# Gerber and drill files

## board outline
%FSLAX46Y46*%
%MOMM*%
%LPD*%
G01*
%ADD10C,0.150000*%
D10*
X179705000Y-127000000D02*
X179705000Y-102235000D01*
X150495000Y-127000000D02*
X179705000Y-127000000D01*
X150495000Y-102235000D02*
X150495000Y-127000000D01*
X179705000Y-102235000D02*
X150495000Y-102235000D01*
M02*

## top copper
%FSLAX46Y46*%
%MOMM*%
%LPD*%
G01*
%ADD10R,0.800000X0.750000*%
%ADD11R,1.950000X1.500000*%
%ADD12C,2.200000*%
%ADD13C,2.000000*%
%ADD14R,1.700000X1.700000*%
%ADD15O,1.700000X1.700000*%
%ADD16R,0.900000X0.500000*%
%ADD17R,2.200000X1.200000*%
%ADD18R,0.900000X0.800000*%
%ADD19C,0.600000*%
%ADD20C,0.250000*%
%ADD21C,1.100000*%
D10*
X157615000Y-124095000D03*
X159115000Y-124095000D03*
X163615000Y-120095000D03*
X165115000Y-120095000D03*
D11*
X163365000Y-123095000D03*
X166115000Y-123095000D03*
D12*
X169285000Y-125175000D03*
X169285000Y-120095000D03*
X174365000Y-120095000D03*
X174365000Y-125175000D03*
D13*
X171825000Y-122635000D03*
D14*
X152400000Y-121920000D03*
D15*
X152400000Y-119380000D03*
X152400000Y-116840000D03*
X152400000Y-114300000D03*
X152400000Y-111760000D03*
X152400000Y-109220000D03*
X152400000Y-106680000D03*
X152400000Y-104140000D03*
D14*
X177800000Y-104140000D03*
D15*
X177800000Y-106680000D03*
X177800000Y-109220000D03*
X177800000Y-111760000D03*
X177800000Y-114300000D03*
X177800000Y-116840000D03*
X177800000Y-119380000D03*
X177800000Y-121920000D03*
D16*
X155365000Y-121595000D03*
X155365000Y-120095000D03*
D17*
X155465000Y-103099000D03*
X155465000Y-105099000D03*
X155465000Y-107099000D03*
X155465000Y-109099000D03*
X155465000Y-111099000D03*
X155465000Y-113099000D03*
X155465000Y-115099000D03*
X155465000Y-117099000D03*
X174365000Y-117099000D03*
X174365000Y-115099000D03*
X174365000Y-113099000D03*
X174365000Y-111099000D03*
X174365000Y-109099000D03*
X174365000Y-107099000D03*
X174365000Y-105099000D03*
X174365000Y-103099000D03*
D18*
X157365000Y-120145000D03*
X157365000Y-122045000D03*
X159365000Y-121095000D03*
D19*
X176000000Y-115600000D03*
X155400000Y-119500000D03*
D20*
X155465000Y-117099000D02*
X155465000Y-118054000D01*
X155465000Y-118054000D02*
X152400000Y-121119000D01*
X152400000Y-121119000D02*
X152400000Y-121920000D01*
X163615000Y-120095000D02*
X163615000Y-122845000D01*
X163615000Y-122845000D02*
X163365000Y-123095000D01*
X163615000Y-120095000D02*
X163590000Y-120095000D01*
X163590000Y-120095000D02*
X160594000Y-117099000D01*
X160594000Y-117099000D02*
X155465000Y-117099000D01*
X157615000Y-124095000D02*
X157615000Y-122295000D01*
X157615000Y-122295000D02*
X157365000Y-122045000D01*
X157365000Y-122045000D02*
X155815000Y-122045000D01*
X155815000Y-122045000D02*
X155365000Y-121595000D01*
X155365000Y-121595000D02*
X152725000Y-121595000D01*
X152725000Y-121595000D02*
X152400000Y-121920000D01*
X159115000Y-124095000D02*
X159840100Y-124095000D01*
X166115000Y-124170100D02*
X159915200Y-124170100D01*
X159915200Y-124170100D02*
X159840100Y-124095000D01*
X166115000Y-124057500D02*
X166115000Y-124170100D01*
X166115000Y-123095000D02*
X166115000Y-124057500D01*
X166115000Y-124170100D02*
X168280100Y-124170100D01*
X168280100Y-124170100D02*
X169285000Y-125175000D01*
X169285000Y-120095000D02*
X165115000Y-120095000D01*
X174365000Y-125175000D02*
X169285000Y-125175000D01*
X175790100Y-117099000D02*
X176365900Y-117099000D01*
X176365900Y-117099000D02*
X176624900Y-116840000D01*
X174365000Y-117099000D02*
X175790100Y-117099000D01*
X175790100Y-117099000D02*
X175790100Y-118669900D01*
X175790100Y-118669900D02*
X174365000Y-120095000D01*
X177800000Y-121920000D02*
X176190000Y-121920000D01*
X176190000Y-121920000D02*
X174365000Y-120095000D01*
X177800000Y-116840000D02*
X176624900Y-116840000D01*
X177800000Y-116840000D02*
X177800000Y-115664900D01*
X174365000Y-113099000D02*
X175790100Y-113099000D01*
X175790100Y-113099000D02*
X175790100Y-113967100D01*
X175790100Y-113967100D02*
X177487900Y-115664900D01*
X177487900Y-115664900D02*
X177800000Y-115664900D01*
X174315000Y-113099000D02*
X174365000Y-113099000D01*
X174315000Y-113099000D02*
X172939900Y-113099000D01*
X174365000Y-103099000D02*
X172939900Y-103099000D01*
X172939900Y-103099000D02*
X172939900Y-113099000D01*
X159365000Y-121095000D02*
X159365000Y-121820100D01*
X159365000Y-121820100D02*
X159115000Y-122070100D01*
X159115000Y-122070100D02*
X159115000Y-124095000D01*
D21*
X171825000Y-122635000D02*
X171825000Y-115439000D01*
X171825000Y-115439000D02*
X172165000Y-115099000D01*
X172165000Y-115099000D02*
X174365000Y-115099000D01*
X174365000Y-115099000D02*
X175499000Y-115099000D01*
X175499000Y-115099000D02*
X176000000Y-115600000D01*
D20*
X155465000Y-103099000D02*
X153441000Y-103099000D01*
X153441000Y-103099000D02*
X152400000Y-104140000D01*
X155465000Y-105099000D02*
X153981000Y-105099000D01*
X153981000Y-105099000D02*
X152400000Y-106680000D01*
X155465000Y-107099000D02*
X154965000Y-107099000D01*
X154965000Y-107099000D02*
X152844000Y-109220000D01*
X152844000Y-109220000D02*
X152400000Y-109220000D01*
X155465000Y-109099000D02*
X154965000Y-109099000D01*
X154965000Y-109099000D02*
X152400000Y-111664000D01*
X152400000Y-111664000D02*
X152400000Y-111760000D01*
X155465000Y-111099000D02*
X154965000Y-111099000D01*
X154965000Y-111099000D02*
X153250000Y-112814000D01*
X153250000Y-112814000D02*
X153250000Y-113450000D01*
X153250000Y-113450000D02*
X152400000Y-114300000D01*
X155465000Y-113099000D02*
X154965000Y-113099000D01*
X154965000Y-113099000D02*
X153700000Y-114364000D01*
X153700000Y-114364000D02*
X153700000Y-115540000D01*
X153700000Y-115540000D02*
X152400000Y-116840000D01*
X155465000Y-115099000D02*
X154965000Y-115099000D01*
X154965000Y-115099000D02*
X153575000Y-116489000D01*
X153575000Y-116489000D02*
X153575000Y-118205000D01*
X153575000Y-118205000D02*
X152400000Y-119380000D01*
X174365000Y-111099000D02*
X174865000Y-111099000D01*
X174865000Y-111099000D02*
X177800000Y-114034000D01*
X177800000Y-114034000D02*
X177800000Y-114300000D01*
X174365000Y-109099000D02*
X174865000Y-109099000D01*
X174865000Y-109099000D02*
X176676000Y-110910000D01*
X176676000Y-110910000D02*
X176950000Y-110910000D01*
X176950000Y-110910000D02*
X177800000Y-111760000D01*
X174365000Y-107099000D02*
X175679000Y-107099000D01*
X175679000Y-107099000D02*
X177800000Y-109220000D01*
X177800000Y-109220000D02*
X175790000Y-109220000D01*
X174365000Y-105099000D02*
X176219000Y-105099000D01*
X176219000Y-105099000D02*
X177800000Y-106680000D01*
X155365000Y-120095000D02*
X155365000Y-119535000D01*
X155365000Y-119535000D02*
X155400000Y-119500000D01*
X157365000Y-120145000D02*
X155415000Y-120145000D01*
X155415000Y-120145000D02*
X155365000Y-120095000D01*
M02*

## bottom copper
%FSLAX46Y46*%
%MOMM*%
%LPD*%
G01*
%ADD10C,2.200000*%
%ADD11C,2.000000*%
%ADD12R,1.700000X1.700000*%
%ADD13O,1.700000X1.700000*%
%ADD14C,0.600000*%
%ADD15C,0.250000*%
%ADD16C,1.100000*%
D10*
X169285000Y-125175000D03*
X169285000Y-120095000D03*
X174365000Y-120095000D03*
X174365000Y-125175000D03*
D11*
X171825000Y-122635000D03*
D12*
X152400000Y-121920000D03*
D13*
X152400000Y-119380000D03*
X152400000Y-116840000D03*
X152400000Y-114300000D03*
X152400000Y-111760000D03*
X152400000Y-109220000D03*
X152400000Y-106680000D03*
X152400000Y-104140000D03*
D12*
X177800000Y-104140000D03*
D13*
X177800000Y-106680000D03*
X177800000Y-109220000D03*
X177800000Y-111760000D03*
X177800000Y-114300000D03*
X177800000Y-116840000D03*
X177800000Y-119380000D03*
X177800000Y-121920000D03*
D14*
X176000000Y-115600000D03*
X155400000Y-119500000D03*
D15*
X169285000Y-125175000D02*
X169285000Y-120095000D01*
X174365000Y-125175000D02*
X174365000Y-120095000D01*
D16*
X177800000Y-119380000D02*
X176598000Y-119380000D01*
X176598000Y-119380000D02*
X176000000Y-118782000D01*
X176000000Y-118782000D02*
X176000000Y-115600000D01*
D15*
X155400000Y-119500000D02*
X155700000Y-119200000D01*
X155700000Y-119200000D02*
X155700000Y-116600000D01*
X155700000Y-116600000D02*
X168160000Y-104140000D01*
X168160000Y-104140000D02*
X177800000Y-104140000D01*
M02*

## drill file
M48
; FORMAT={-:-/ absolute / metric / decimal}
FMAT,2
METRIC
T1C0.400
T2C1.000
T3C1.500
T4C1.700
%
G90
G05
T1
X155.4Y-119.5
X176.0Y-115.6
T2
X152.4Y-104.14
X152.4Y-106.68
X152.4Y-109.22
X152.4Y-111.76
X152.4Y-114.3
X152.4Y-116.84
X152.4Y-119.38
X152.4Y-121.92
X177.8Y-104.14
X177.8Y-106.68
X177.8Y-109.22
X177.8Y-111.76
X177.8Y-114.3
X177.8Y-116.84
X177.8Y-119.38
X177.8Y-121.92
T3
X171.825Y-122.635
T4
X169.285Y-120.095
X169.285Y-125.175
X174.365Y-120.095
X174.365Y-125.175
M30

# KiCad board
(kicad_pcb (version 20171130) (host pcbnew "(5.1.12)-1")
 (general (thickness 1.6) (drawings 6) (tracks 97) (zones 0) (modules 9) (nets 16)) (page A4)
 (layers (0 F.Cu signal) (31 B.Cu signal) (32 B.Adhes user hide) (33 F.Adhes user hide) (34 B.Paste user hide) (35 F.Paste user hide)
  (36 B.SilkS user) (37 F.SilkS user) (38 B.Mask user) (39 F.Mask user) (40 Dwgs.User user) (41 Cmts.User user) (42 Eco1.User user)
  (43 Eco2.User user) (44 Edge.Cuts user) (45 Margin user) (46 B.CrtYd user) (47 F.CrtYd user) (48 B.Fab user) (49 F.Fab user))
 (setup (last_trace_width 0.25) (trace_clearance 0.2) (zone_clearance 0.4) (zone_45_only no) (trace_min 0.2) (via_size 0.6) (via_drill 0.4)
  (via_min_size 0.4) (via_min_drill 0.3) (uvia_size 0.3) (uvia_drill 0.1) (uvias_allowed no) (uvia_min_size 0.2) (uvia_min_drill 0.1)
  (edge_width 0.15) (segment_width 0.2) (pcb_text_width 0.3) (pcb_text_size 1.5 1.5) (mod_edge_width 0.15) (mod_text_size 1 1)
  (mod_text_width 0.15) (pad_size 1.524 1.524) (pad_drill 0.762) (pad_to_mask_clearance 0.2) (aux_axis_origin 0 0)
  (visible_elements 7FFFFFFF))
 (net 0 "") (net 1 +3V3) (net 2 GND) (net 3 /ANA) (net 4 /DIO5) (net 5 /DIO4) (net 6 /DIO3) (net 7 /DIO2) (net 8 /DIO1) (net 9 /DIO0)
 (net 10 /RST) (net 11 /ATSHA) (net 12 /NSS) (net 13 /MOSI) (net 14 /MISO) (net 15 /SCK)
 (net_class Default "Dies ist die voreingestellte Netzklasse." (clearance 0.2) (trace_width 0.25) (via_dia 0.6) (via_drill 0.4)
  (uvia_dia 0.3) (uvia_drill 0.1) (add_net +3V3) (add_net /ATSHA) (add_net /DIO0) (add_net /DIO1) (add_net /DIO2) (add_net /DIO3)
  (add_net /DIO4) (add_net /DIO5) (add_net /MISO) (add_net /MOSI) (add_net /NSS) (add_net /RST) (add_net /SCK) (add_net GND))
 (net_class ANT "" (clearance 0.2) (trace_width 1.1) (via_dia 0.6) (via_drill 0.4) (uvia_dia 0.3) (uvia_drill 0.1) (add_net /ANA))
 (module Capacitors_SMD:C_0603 (layer F.Cu) (at 158.365 124.095)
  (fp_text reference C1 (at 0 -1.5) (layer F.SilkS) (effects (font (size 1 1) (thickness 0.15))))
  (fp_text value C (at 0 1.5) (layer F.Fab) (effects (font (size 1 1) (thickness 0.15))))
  (pad 1 smd rect (at -0.75 0) (size 0.8 0.75) (layers F.Cu F.Paste F.Mask) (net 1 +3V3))
  (pad 2 smd rect (at 0.75 0) (size 0.8 0.75) (layers F.Cu F.Paste F.Mask) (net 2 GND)))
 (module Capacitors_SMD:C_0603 (layer F.Cu) (at 164.365 120.095)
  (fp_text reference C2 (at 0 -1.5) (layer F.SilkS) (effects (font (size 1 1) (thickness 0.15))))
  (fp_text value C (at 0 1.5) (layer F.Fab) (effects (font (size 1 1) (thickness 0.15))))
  (pad 1 smd rect (at -0.75 0) (size 0.8 0.75) (layers F.Cu F.Paste F.Mask) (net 1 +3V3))
  (pad 2 smd rect (at 0.75 0) (size 0.8 0.75) (layers F.Cu F.Paste F.Mask) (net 2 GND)))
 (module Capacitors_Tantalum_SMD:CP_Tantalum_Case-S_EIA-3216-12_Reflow (layer F.Cu) (at 164.74 123.095)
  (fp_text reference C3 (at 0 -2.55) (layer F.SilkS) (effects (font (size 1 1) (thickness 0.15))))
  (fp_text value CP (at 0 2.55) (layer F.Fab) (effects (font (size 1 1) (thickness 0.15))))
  (pad 1 smd rect (at -1.375 0) (size 1.95 1.5) (layers F.Cu F.Paste F.Mask) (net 1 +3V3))
  (pad 2 smd rect (at 1.375 0) (size 1.95 1.5) (layers F.Cu F.Paste F.Mask) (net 2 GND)))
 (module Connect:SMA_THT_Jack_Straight (layer F.Cu) (at 171.825 122.635)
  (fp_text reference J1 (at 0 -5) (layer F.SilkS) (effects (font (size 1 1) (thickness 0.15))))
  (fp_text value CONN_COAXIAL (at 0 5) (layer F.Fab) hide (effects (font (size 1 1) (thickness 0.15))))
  (pad 2 thru_hole circle (at -2.54 2.54) (size 2.2 2.2) (drill 1.7) (layers *.Cu *.Mask) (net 2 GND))
  (pad 2 thru_hole circle (at -2.54 -2.54) (size 2.2 2.2) (drill 1.7) (layers *.Cu *.Mask) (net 2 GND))
  (pad 2 thru_hole circle (at 2.54 -2.54) (size 2.2 2.2) (drill 1.7) (layers *.Cu *.Mask) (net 2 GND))
  (pad 2 thru_hole circle (at 2.54 2.54) (size 2.2 2.2) (drill 1.7) (layers *.Cu *.Mask) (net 2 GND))
  (pad 1 thru_hole circle (at 0 0) (size 2 2) (drill 1.5) (layers *.Cu *.Mask) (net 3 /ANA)))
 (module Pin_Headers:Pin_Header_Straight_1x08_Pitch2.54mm (layer F.Cu) (at 152.4 121.92 180)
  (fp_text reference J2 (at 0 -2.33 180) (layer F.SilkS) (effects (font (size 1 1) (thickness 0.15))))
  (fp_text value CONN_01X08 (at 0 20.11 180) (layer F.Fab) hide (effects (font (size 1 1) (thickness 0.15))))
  (pad 1 thru_hole rect (at 0 0 180) (size 1.7 1.7) (drill 1) (layers *.Cu *.Mask) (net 1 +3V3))
  (pad 2 thru_hole oval (at 0 2.54 180) (size 1.7 1.7) (drill 1) (layers *.Cu *.Mask) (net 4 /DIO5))
  (pad 3 thru_hole oval (at 0 5.08 180) (size 1.7 1.7) (drill 1) (layers *.Cu *.Mask) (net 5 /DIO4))
  (pad 4 thru_hole oval (at 0 7.62 180) (size 1.7 1.7) (drill 1) (layers *.Cu *.Mask) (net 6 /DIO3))
  (pad 5 thru_hole oval (at 0 10.16 180) (size 1.7 1.7) (drill 1) (layers *.Cu *.Mask) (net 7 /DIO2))
  (pad 6 thru_hole oval (at 0 12.7 180) (size 1.7 1.7) (drill 1) (layers *.Cu *.Mask) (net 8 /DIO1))
  (pad 7 thru_hole oval (at 0 15.24 180) (size 1.7 1.7) (drill 1) (layers *.Cu *.Mask) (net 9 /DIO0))
  (pad 8 thru_hole oval (at 0 17.78 180) (size 1.7 1.7) (drill 1) (layers *.Cu *.Mask) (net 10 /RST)))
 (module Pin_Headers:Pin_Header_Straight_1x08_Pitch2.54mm (layer F.Cu) (at 177.8 104.14)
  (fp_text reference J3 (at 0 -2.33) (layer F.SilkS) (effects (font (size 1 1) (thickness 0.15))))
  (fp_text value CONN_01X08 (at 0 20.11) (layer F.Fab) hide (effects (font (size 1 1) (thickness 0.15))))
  (pad 1 thru_hole rect (at 0 0) (size 1.7 1.7) (drill 1) (layers *.Cu *.Mask) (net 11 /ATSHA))
  (pad 2 thru_hole oval (at 0 2.54) (size 1.7 1.7) (drill 1) (layers *.Cu *.Mask) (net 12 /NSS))
  (pad 3 thru_hole oval (at 0 5.08) (size 1.7 1.7) (drill 1) (layers *.Cu *.Mask) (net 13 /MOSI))
  (pad 4 thru_hole oval (at 0 7.62) (size 1.7 1.7) (drill 1) (layers *.Cu *.Mask) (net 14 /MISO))
  (pad 5 thru_hole oval (at 0 10.16) (size 1.7 1.7) (drill 1) (layers *.Cu *.Mask) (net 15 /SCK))
  (pad 6 thru_hole oval (at 0 12.7) (size 1.7 1.7) (drill 1) (layers *.Cu *.Mask) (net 2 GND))
  (pad 7 thru_hole oval (at 0 15.24) (size 1.7 1.7) (drill 1) (layers *.Cu *.Mask) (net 3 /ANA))
  (pad 8 thru_hole oval (at 0 17.78) (size 1.7 1.7) (drill 1) (layers *.Cu *.Mask) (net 2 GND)))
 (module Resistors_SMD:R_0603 (layer F.Cu) (at 155.365 120.845 90)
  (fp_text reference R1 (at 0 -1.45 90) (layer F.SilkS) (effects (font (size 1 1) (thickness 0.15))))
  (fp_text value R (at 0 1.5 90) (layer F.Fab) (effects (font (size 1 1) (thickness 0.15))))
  (pad 1 smd rect (at -0.75 0 90) (size 0.5 0.9) (layers F.Cu F.Paste F.Mask) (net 1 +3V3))
  (pad 2 smd rect (at 0.75 0 90) (size 0.5 0.9) (layers F.Cu F.Paste F.Mask) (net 11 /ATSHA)))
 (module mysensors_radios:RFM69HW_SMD (layer F.Cu) (at 156.465 103.099)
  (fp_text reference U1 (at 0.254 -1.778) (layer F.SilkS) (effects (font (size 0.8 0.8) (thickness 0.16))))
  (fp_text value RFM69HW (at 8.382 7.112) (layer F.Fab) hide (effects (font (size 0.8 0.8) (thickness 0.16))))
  (pad 1 smd rect (at -1 0) (size 2.2 1.2) (layers F.Cu F.Paste F.Mask) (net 10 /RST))
  (pad 2 smd rect (at -1 2) (size 2.2 1.2) (layers F.Cu F.Paste F.Mask) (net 9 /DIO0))
  (pad 3 smd rect (at -1 4) (size 2.2 1.2) (layers F.Cu F.Paste F.Mask) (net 8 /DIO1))
  (pad 4 smd rect (at -1 6) (size 2.2 1.2) (layers F.Cu F.Paste F.Mask) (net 7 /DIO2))
  (pad 5 smd rect (at -1 8) (size 2.2 1.2) (layers F.Cu F.Paste F.Mask) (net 6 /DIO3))
  (pad 6 smd rect (at -1 10) (size 2.2 1.2) (layers F.Cu F.Paste F.Mask) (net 5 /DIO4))
  (pad 7 smd rect (at -1 12) (size 2.2 1.2) (layers F.Cu F.Paste F.Mask) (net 4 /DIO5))
  (pad 8 smd rect (at -1 14) (size 2.2 1.2) (layers F.Cu F.Paste F.Mask) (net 1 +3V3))
  (pad 9 smd rect (at 17.9 14) (size 2.2 1.2) (layers F.Cu F.Paste F.Mask) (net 2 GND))
  (pad 10 smd rect (at 17.9 12) (size 2.2 1.2) (layers F.Cu F.Paste F.Mask) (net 3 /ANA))
  (pad 11 smd rect (at 17.9 10) (size 2.2 1.2) (layers F.Cu F.Paste F.Mask) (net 2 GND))
  (pad 12 smd rect (at 17.9 8) (size 2.2 1.2) (layers F.Cu F.Paste F.Mask) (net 15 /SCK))
  (pad 13 smd rect (at 17.9 6) (size 2.2 1.2) (layers F.Cu F.Paste F.Mask) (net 14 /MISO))
  (pad 14 smd rect (at 17.9 4) (size 2.2 1.2) (layers F.Cu F.Paste F.Mask) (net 13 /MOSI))
  (pad 15 smd rect (at 17.9 2) (size 2.2 1.2) (layers F.Cu F.Paste F.Mask) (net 12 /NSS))
  (pad 16 smd rect (at 17.9 0) (size 2.2 1.2) (layers F.Cu F.Paste F.Mask) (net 2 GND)))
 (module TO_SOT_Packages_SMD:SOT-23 (layer F.Cu) (at 158.365 121.095)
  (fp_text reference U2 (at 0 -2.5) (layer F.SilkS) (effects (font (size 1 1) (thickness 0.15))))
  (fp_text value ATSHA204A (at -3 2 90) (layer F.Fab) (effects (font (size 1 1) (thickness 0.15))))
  (pad 1 smd rect (at -1 -0.95) (size 0.9 0.8) (layers F.Cu F.Paste F.Mask) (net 11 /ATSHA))
  (pad 2 smd rect (at -1 0.95) (size 0.9 0.8) (layers F.Cu F.Paste F.Mask) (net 1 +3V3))
  (pad 3 smd rect (at 1 0) (size 0.9 0.8) (layers F.Cu F.Paste F.Mask) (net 2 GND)))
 (gr_line (start 179.705 127) (end 179.705 102.235) (layer Edge.Cuts) (width 0.15))
 (gr_line (start 150.495 127) (end 179.705 127) (layer Edge.Cuts) (width 0.15))
 (gr_line (start 150.495 102.235) (end 150.495 127) (layer Edge.Cuts) (width 0.15))
 (gr_line (start 179.705 102.235) (end 150.495 102.235) (layer Edge.Cuts) (width 0.15))
 (segment (start 155.465 117.099) (end 155.465 118.054) (width 0.25) (layer F.Cu) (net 1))
 (segment (start 155.465 118.054) (end 152.4 121.119) (width 0.25) (layer F.Cu) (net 1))
 (segment (start 152.4 121.119) (end 152.4 121.92) (width 0.25) (layer F.Cu) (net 1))
 (segment (start 163.615 120.095) (end 163.615 122.845) (width 0.25) (layer F.Cu) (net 1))
 (segment (start 163.615 122.845) (end 163.365 123.095) (width 0.25) (layer F.Cu) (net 1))
 (segment (start 163.615 120.095) (end 163.59 120.095) (width 0.25) (layer F.Cu) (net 1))
 (segment (start 163.59 120.095) (end 160.594 117.099) (width 0.25) (layer F.Cu) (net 1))
 (segment (start 160.594 117.099) (end 155.465 117.099) (width 0.25) (layer F.Cu) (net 1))
 (segment (start 157.615 124.095) (end 157.615 122.295) (width 0.25) (layer F.Cu) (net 1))
 (segment (start 157.615 122.295) (end 157.365 122.045) (width 0.25) (layer F.Cu) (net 1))
 (segment (start 157.365 122.045) (end 155.815 122.045) (width 0.25) (layer F.Cu) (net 1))
 (segment (start 155.815 122.045) (end 155.365 121.595) (width 0.25) (layer F.Cu) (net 1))
 (segment (start 155.365 121.595) (end 152.725 121.595) (width 0.25) (layer F.Cu) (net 1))
 (segment (start 152.725 121.595) (end 152.4 121.92) (width 0.25) (layer F.Cu) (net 1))
 (segment (start 159.115 124.095) (end 159.8401 124.095) (width 0.25) (layer F.Cu) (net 2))
 (segment (start 166.115 124.1701) (end 159.9152 124.1701) (width 0.25) (layer F.Cu) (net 2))
 (segment (start 159.9152 124.1701) (end 159.8401 124.095) (width 0.25) (layer F.Cu) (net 2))
 (segment (start 166.115 124.0575) (end 166.115 124.1701) (width 0.25) (layer F.Cu) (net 2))
 (segment (start 166.115 123.095) (end 166.115 124.0575) (width 0.25) (layer F.Cu) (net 2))
 (segment (start 166.115 124.1701) (end 168.2801 124.1701) (width 0.25) (layer F.Cu) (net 2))
 (segment (start 168.2801 124.1701) (end 169.285 125.175) (width 0.25) (layer F.Cu) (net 2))
 (segment (start 169.285 125.175) (end 169.285 120.095) (width 0.25) (layer B.Cu) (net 2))
 (segment (start 169.285 120.095) (end 165.115 120.095) (width 0.25) (layer F.Cu) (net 2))
 (segment (start 174.365 125.175) (end 169.285 125.175) (width 0.25) (layer F.Cu) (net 2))
 (segment (start 174.365 125.175) (end 174.365 120.095) (width 0.25) (layer B.Cu) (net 2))
 (segment (start 175.7901 117.099) (end 176.3659 117.099) (width 0.25) (layer F.Cu) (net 2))
 (segment (start 176.3659 117.099) (end 176.6249 116.84) (width 0.25) (layer F.Cu) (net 2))
 (segment (start 174.365 117.099) (end 175.7901 117.099) (width 0.25) (layer F.Cu) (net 2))
 (segment (start 175.7901 117.099) (end 175.7901 118.6699) (width 0.25) (layer F.Cu) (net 2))
 (segment (start 175.7901 118.6699) (end 174.365 120.095) (width 0.25) (layer F.Cu) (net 2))
 (segment (start 177.8 121.92) (end 176.19 121.92) (width 0.25) (layer F.Cu) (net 2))
 (segment (start 176.19 121.92) (end 174.365 120.095) (width 0.25) (layer F.Cu) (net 2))
 (segment (start 177.8 116.84) (end 176.6249 116.84) (width 0.25) (layer F.Cu) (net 2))
 (segment (start 177.8 116.84) (end 177.8 115.6649) (width 0.25) (layer F.Cu) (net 2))
 (segment (start 174.365 113.099) (end 175.7901 113.099) (width 0.25) (layer F.Cu) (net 2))
 (segment (start 175.7901 113.099) (end 175.7901 113.9671) (width 0.25) (layer F.Cu) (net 2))
 (segment (start 175.7901 113.9671) (end 177.4879 115.6649) (width 0.25) (layer F.Cu) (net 2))
 (segment (start 177.4879 115.6649) (end 177.8 115.6649) (width 0.25) (layer F.Cu) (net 2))
 (segment (start 174.315 113.099) (end 174.365 113.099) (width 0.25) (layer F.Cu) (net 2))
 (segment (start 174.315 113.099) (end 172.9399 113.099) (width 0.25) (layer F.Cu) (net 2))
 (segment (start 174.365 103.099) (end 172.9399 103.099) (width 0.25) (layer F.Cu) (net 2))
 (segment (start 172.9399 103.099) (end 172.9399 113.099) (width 0.25) (layer F.Cu) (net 2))
 (segment (start 159.365 121.095) (end 159.365 121.8201) (width 0.25) (layer F.Cu) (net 2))
 (segment (start 159.365 121.8201) (end 159.115 122.0701) (width 0.25) (layer F.Cu) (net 2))
 (segment (start 159.115 122.0701) (end 159.115 124.095) (width 0.25) (layer F.Cu) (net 2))
 (segment (start 171.825 122.635) (end 171.825 115.439) (width 1.1) (layer F.Cu) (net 3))
 (segment (start 171.825 115.439) (end 172.165 115.099) (width 1.1) (layer F.Cu) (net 3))
 (segment (start 172.165 115.099) (end 174.365 115.099) (width 1.1) (layer F.Cu) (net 3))
 (segment (start 174.365 115.099) (end 175.499 115.099) (width 1.1) (layer F.Cu) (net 3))
 (segment (start 175.499 115.099) (end 176 115.6) (width 1.1) (layer F.Cu) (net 3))
 (segment (start 177.8 119.38) (end 176.598 119.38) (width 1.1) (layer B.Cu) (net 3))
 (segment (start 176.598 119.38) (end 176 118.782) (width 1.1) (layer B.Cu) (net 3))
 (segment (start 176 118.782) (end 176 115.6) (width 1.1) (layer B.Cu) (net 3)) (via (at 176 115.6) (size 0.6) (layers F.Cu B.Cu) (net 3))
 (segment (start 155.465 103.099) (end 153.441 103.099) (width 0.25) (layer F.Cu) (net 10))
 (segment (start 153.441 103.099) (end 152.4 104.14) (width 0.25) (layer F.Cu) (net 10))
 (segment (start 155.465 105.099) (end 153.981 105.099) (width 0.25) (layer F.Cu) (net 9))
 (segment (start 153.981 105.099) (end 152.4 106.68) (width 0.25) (layer F.Cu) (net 9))
 (segment (start 155.465 107.099) (end 154.965 107.099) (width 0.25) (layer F.Cu) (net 8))
 (segment (start 154.965 107.099) (end 152.844 109.22) (width 0.25) (layer F.Cu) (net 8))
 (segment (start 152.844 109.22) (end 152.4 109.22) (width 0.25) (layer F.Cu) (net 8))
 (segment (start 155.465 109.099) (end 154.965 109.099) (width 0.25) (layer F.Cu) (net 7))
 (segment (start 154.965 109.099) (end 152.4 111.664) (width 0.25) (layer F.Cu) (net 7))
 (segment (start 152.4 111.664) (end 152.4 111.76) (width 0.25) (layer F.Cu) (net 7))
 (segment (start 155.465 111.099) (end 154.965 111.099) (width 0.25) (layer F.Cu) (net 6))
 (segment (start 154.965 111.099) (end 153.25 112.814) (width 0.25) (layer F.Cu) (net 6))
 (segment (start 153.25 112.814) (end 153.25 113.45) (width 0.25) (layer F.Cu) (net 6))
 (segment (start 153.25 113.45) (end 152.4 114.3) (width 0.25) (layer F.Cu) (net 6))
 (segment (start 155.465 113.099) (end 154.965 113.099) (width 0.25) (layer F.Cu) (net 5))
 (segment (start 154.965 113.099) (end 153.7 114.364) (width 0.25) (layer F.Cu) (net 5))
 (segment (start 153.7 114.364) (end 153.7 115.54) (width 0.25) (layer F.Cu) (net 5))
 (segment (start 153.7 115.54) (end 152.4 116.84) (width 0.25) (layer F.Cu) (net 5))
 (segment (start 155.465 115.099) (end 154.965 115.099) (width 0.25) (layer F.Cu) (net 4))
 (segment (start 154.965 115.099) (end 153.575 116.489) (width 0.25) (layer F.Cu) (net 4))
 (segment (start 153.575 116.489) (end 153.575 118.205) (width 0.25) (layer F.Cu) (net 4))
 (segment (start 153.575 118.205) (end 152.4 119.38) (width 0.25) (layer F.Cu) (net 4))
 (segment (start 174.365 111.099) (end 174.865 111.099) (width 0.25) (layer F.Cu) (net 15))
 (segment (start 174.865 111.099) (end 177.8 114.034) (width 0.25) (layer F.Cu) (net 15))
 (segment (start 177.8 114.034) (end 177.8 114.3) (width 0.25) (layer F.Cu) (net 15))
 (segment (start 174.365 109.099) (end 174.865 109.099) (width 0.25) (layer F.Cu) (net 14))
 (segment (start 174.865 109.099) (end 176.676 110.91) (width 0.25) (layer F.Cu) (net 14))
 (segment (start 176.676 110.91) (end 176.95 110.91) (width 0.25) (layer F.Cu) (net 14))
 (segment (start 176.95 110.91) (end 177.8 111.76) (width 0.25) (layer F.Cu) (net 14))
 (segment (start 174.365 107.099) (end 175.679 107.099) (width 0.25) (layer F.Cu) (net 13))
 (segment (start 175.679 107.099) (end 177.8 109.22) (width 0.25) (layer F.Cu) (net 13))
 (segment (start 177.8 109.22) (end 175.79 109.22) (width 0.25) (layer F.Cu) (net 13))
 (segment (start 174.365 105.099) (end 176.219 105.099) (width 0.25) (layer F.Cu) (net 12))
 (segment (start 176.219 105.099) (end 177.8 106.68) (width 0.25) (layer F.Cu) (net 12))
 (segment (start 155.365 120.095) (end 155.365 119.535) (width 0.25) (layer F.Cu) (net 11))
 (segment (start 155.365 119.535) (end 155.4 119.5) (width 0.25) (layer F.Cu) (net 11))
 (segment (start 155.4 119.5) (end 155.7 119.2) (width 0.25) (layer B.Cu) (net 11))
 (segment (start 155.7 119.2) (end 155.7 116.6) (width 0.25) (layer B.Cu) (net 11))
 (segment (start 155.7 116.6) (end 168.16 104.14) (width 0.25) (layer B.Cu) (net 11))
 (segment (start 168.16 104.14) (end 177.8 104.14) (width 0.25) (layer B.Cu) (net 11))
 (segment (start 157.365 120.145) (end 155.415 120.145) (width 0.25) (layer F.Cu) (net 11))
 (segment (start 155.415 120.145) (end 155.365 120.095) (width 0.25) (layer F.Cu) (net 11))
 (via (at 155.4 119.5) (size 0.6) (layers F.Cu B.Cu) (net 11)))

